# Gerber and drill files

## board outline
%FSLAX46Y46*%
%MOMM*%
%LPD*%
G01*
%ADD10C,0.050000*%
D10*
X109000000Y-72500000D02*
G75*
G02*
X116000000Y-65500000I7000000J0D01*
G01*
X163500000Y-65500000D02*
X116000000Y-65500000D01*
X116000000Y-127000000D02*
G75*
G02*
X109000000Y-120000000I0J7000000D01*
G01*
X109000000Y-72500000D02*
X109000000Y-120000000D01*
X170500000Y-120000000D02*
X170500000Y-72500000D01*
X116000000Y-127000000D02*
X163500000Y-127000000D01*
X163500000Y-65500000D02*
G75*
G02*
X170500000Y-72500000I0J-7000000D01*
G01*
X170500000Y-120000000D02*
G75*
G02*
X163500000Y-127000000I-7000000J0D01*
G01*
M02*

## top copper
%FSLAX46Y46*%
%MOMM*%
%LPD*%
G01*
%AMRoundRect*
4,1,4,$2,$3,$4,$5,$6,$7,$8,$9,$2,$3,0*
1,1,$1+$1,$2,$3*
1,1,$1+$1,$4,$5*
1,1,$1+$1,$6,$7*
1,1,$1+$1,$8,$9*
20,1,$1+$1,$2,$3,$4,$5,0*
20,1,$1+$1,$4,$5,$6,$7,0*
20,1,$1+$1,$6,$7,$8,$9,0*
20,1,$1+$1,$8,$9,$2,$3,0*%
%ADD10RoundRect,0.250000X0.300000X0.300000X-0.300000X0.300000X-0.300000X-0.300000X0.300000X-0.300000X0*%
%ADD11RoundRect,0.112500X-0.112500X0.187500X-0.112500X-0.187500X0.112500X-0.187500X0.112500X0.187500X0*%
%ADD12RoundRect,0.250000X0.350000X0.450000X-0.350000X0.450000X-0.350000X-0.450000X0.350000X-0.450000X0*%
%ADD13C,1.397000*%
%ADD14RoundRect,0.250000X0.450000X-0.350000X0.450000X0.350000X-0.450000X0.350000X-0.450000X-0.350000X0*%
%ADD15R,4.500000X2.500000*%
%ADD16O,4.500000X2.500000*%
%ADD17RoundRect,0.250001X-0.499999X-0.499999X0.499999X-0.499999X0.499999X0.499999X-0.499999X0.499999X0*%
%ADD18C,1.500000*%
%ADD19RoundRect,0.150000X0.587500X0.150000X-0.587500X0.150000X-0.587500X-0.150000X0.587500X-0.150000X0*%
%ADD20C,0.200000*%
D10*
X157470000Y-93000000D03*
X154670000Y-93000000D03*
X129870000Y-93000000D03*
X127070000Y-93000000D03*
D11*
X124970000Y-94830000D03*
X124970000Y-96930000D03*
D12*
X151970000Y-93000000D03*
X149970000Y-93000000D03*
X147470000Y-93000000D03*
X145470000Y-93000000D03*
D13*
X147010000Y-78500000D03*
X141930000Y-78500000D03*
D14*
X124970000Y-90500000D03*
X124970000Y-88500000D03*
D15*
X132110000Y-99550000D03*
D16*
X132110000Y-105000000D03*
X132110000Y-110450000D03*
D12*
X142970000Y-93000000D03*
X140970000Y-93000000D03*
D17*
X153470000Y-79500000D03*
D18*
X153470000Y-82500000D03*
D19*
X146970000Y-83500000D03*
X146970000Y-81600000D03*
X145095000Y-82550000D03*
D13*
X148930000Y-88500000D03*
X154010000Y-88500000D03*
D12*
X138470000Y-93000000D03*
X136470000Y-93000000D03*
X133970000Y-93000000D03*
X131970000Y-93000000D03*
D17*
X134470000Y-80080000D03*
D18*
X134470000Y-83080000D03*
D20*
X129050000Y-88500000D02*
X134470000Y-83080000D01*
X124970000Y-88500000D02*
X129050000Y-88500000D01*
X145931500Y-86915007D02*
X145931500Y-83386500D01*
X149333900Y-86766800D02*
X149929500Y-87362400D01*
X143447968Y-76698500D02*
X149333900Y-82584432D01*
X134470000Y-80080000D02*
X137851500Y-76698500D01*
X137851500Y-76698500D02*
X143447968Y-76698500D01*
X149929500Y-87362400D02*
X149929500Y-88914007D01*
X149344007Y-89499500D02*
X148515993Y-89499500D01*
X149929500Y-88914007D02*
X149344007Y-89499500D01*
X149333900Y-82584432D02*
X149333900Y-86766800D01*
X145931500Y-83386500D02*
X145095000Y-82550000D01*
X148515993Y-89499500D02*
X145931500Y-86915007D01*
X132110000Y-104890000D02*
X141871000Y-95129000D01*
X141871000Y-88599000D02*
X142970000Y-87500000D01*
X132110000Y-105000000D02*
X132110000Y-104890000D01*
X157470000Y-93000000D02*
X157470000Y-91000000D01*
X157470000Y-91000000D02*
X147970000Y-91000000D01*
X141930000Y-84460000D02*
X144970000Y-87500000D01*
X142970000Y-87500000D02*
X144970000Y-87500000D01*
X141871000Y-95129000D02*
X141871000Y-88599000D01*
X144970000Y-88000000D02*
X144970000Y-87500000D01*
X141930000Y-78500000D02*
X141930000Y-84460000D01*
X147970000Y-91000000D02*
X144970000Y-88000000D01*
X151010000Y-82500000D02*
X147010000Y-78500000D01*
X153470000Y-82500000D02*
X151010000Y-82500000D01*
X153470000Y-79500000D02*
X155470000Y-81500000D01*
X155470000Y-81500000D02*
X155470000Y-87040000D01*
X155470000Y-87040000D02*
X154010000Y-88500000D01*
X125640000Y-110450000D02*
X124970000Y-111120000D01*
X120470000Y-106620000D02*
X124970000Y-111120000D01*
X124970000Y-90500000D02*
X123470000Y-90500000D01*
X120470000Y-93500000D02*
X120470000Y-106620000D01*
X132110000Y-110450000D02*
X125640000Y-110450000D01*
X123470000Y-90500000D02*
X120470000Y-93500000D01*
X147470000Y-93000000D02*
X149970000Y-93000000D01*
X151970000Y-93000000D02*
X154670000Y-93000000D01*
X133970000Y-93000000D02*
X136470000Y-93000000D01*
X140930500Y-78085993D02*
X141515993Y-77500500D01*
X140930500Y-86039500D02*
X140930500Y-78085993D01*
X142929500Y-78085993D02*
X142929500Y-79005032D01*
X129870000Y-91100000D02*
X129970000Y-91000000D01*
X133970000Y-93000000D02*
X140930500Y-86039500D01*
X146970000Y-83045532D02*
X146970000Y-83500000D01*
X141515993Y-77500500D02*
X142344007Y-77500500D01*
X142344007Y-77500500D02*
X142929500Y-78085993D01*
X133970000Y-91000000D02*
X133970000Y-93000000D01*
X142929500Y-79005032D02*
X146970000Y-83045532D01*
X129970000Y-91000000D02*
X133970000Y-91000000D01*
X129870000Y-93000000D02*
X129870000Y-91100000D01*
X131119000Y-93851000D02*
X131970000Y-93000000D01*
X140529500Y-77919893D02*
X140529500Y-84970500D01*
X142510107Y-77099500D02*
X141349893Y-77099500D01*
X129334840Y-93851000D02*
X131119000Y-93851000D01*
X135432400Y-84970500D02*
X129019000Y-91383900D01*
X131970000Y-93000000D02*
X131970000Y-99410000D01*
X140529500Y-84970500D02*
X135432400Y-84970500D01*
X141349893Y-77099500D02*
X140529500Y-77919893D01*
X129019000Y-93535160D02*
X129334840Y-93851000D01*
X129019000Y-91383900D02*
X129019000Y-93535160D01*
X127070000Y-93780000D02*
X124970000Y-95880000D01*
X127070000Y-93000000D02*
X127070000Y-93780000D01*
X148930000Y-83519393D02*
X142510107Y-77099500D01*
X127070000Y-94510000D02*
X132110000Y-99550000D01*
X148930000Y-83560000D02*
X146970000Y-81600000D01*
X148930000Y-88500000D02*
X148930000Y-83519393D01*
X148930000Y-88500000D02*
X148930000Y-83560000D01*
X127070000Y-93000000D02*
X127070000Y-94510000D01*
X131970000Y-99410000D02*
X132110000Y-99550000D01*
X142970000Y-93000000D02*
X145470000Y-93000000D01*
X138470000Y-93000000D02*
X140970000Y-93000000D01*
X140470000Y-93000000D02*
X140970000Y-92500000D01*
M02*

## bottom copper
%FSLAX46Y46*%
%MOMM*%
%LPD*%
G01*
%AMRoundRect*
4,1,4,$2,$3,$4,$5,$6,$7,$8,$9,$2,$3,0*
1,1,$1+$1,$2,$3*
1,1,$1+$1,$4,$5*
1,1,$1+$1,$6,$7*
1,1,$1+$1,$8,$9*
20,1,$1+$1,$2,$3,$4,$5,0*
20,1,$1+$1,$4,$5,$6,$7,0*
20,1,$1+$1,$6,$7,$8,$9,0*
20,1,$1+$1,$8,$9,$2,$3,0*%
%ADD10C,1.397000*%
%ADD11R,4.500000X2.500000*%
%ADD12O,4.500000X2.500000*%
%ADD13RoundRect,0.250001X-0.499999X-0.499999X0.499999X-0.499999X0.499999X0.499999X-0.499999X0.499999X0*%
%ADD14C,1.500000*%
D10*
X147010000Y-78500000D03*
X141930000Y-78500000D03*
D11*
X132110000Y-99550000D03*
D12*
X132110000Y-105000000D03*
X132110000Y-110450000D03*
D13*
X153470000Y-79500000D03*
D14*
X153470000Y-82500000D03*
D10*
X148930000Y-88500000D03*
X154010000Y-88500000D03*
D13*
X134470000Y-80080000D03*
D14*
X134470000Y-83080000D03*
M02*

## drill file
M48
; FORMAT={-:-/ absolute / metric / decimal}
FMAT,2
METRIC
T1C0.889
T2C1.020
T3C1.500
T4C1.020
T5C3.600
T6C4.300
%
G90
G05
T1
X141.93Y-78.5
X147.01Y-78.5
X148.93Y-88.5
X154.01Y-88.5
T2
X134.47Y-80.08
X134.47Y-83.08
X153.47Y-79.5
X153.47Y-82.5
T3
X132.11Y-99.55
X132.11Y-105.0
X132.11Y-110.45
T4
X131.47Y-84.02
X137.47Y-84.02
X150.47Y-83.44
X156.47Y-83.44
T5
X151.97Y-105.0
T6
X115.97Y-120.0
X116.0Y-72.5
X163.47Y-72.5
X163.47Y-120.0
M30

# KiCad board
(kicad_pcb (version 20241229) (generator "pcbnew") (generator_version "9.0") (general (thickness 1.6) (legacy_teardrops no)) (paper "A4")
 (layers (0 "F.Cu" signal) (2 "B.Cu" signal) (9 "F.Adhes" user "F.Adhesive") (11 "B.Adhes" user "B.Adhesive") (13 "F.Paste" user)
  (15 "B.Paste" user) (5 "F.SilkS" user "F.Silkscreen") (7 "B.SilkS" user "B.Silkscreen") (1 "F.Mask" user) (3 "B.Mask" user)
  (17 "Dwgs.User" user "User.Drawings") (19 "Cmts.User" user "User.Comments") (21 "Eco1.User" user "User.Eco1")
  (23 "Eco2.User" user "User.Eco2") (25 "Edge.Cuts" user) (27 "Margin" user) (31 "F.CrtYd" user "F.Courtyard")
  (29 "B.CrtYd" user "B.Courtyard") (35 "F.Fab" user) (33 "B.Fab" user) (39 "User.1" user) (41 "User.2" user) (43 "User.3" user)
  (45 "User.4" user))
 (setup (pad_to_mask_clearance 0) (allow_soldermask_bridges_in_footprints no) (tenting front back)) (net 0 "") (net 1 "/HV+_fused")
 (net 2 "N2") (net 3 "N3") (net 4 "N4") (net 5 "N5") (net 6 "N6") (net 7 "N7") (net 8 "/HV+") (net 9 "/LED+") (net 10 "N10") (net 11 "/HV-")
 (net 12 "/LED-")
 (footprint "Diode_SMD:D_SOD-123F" (layer "F.Cu") (at 156.07 93 180)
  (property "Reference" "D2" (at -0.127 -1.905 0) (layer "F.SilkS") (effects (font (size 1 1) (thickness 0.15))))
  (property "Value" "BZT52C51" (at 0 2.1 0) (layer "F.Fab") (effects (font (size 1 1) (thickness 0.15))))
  (pad "1" smd roundrect (at -1.4 0 180) (size 1.1 1.1) (layers "F.Cu" "F.Mask" "F.Paste") (roundrect_rratio 0.2272727273)
   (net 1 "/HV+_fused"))
  (pad "2" smd roundrect (at 1.4 0 180) (size 1.1 1.1) (layers "F.Cu" "F.Mask" "F.Paste") (roundrect_rratio 0.2272727273) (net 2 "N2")))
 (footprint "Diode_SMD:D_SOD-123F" (layer "F.Cu") (at 128.47 93 180)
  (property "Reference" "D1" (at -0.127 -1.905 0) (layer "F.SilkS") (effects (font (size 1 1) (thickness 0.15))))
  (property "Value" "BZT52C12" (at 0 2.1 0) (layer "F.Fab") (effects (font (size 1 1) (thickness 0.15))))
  (pad "1" smd roundrect (at -1.4 0 180) (size 1.1 1.1) (layers "F.Cu" "F.Mask" "F.Paste") (roundrect_rratio 0.2272727273) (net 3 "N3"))
  (pad "2" smd roundrect (at 1.4 0 180) (size 1.1 1.1) (layers "F.Cu" "F.Mask" "F.Paste") (roundrect_rratio 0.2272727273) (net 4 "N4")))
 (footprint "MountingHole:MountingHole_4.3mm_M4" (layer "F.Cu") (at 116 72.5)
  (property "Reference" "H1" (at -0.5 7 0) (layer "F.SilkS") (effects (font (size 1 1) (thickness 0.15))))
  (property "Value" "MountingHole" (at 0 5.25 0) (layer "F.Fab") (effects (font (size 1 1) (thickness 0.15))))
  (pad "" np_thru_hole circle (at 0 0) (size 4.3 4.3) (drill 4.3) (layers "*.Cu" "*.Mask")))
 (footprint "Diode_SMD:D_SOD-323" (layer "F.Cu") (at 124.97 95.88 -90)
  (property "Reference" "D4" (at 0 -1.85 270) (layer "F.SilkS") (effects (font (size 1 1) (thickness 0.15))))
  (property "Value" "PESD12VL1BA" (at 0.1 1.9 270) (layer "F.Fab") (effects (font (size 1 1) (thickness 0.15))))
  (pad "1" smd roundrect (at -1.05 0 270) (size 0.6 0.45) (layers "F.Cu" "F.Mask" "F.Paste") (roundrect_rratio 0.25) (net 4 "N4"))
  (pad "2" smd roundrect (at 1.05 0 270) (size 0.6 0.45) (layers "F.Cu" "F.Mask" "F.Paste") (roundrect_rratio 0.25) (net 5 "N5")))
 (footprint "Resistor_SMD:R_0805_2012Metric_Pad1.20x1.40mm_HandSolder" (layer "F.Cu") (at 150.97 93 180)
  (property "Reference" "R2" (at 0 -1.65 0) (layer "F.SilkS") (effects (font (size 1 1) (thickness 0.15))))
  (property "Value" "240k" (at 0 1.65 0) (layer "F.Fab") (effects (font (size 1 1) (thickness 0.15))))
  (pad "1" smd roundrect (at -1 0 180) (size 1.2 1.4) (layers "F.Cu" "F.Mask" "F.Paste") (roundrect_rratio 0.208333) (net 2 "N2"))
  (pad "2" smd roundrect (at 1 0 180) (size 1.2 1.4) (layers "F.Cu" "F.Mask" "F.Paste") (roundrect_rratio 0.208333) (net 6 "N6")))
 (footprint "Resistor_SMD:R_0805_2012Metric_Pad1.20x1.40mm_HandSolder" (layer "F.Cu") (at 146.47 93 180)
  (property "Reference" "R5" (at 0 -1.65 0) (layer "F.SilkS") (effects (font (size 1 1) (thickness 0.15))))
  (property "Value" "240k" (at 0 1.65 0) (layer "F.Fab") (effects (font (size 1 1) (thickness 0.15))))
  (pad "1" smd roundrect (at -1 0 180) (size 1.2 1.4) (layers "F.Cu" "F.Mask" "F.Paste") (roundrect_rratio 0.208333) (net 6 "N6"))
  (pad "2" smd roundrect (at 1 0 180) (size 1.2 1.4) (layers "F.Cu" "F.Mask" "F.Paste") (roundrect_rratio 0.208333) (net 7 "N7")))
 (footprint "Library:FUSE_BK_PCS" (layer "F.Cu") (at 144.47 78.5 180)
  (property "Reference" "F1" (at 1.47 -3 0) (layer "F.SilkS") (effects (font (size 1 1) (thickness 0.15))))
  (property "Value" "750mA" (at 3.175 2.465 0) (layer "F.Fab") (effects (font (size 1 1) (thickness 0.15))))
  (pad "1" thru_hole circle (at -2.54 0 180) (size 1.397 1.397) (drill 0.889) (layers "*.Cu" "*.Mask") (remove_unused_layers no)
   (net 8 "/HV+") (solder_mask_margin 0.102))
  (pad "2" thru_hole circle (at 2.54 0 180) (size 1.397 1.397) (drill 0.889) (layers "*.Cu" "*.Mask") (remove_unused_layers no)
   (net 1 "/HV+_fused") (solder_mask_margin 0.102)))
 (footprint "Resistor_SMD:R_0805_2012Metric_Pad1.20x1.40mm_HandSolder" (layer "F.Cu") (at 124.97 89.5 90)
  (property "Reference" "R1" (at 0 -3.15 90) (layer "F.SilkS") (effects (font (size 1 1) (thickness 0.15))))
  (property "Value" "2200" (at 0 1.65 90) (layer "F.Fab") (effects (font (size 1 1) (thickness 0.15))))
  (pad "1" smd roundrect (at -1 0 90) (size 1.2 1.4) (layers "F.Cu" "F.Mask" "F.Paste") (roundrect_rratio 0.208333) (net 5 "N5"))
  (pad "2" smd roundrect (at 1 0 90) (size 1.2 1.4) (layers "F.Cu" "F.Mask" "F.Paste") (roundrect_rratio 0.208333) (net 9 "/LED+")))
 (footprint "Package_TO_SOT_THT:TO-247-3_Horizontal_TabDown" (layer "F.Cu") (at 132.11 99.55 -90)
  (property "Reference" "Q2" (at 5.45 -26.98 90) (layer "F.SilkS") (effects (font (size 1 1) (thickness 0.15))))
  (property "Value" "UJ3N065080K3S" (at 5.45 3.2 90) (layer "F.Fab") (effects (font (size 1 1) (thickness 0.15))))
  (pad "" np_thru_hole circle (at 5.45 -19.86 270) (size 3.6 3.6) (drill 3.6) (layers "*.Cu" "*.Mask"))
  (pad "1" thru_hole rect (at 0 0 270) (size 2.5 4.5) (drill 1.5) (layers "*.Cu" "*.Mask") (remove_unused_layers no) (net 4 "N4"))
  (pad "2" thru_hole oval (at 5.45 0 270) (size 2.5 4.5) (drill 1.5) (layers "*.Cu" "*.Mask") (remove_unused_layers no) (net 1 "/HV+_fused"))
  (pad "3" thru_hole oval (at 10.9 0 270) (size 2.5 4.5) (drill 1.5) (layers "*.Cu" "*.Mask") (remove_unused_layers no) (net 5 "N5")))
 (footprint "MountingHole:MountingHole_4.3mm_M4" (layer "F.Cu") (at 115.97 120)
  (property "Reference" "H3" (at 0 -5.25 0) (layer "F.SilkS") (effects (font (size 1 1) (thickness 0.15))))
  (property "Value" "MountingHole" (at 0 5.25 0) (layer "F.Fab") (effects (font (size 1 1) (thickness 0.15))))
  (pad "" np_thru_hole circle (at 0 0) (size 4.3 4.3) (drill 4.3) (layers "*.Cu" "*.Mask")))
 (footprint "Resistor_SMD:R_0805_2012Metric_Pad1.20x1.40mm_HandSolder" (layer "F.Cu") (at 141.97 93 180)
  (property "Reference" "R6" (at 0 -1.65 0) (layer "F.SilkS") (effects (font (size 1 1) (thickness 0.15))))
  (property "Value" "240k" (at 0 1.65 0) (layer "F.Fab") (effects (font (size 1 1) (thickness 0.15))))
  (pad "1" smd roundrect (at -1 0 180) (size 1.2 1.4) (layers "F.Cu" "F.Mask" "F.Paste") (roundrect_rratio 0.208333) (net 7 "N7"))
  (pad "2" smd roundrect (at 1 0 180) (size 1.2 1.4) (layers "F.Cu" "F.Mask" "F.Paste") (roundrect_rratio 0.208333) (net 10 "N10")))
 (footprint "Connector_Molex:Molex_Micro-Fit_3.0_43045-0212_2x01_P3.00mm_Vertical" (layer "F.Cu") (at 153.47 79.5)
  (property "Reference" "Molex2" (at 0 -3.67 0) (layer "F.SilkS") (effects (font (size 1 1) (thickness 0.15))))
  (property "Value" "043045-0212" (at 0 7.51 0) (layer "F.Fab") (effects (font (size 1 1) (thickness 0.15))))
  (pad "" np_thru_hole circle (at -3 3.94) (size 1.02 1.02) (drill 1.02) (layers "*.Cu" "*.Mask"))
  (pad "" np_thru_hole circle (at 3 3.94) (size 1.02 1.02) (drill 1.02) (layers "*.Cu" "*.Mask"))
  (pad "1" thru_hole roundrect (at 0 0) (size 1.5 1.5) (drill 1.02) (layers "*.Cu" "*.Mask") (remove_unused_layers no)
   (roundrect_rratio 0.166667) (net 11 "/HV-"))
  (pad "2" thru_hole circle (at 0 3) (size 1.5 1.5) (drill 1.02) (layers "*.Cu" "*.Mask") (remove_unused_layers no) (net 8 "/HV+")))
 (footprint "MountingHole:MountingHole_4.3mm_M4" (layer "F.Cu") (at 163.47 72.5)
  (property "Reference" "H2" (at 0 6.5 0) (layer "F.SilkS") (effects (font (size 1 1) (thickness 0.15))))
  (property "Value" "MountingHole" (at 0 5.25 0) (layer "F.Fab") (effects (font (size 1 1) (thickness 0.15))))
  (pad "" np_thru_hole circle (at 0 0) (size 4.3 4.3) (drill 4.3) (layers "*.Cu" "*.Mask")))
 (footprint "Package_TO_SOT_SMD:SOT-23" (layer "F.Cu") (at 146.0325 82.55 180)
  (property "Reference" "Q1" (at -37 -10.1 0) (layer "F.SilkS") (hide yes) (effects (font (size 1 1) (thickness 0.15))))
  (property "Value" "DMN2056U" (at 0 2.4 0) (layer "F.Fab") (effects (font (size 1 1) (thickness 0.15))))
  (pad "1" smd roundrect (at -0.9375 -0.95 180) (size 1.475 0.6) (layers "F.Cu" "F.Mask" "F.Paste") (roundrect_rratio 0.25) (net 3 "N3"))
  (pad "2" smd roundrect (at -0.9375 0.95 180) (size 1.475 0.6) (layers "F.Cu" "F.Mask" "F.Paste") (roundrect_rratio 0.25) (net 4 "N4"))
  (pad "3" smd roundrect (at 0.9375 0 180) (size 1.475 0.6) (layers "F.Cu" "F.Mask" "F.Paste") (roundrect_rratio 0.25) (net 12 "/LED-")))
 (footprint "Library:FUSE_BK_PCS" (layer "F.Cu") (at 151.47 88.5)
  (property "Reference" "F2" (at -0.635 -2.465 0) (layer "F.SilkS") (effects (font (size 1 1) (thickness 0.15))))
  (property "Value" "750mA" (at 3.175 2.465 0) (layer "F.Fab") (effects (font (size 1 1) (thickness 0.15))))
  (pad "1" thru_hole circle (at -2.54 0) (size 1.397 1.397) (drill 0.889) (layers "*.Cu" "*.Mask") (remove_unused_layers no) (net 4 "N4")
   (solder_mask_margin 0.102))
  (pad "2" thru_hole circle (at 2.54 0) (size 1.397 1.397) (drill 0.889) (layers "*.Cu" "*.Mask") (remove_unused_layers no) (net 11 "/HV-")
   (solder_mask_margin 0.102)))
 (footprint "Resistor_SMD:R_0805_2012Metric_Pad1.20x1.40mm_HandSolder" (layer "F.Cu") (at 137.47 93 180)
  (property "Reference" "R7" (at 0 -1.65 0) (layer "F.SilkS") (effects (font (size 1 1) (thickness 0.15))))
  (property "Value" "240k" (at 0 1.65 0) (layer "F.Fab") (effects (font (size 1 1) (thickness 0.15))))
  (pad "1" smd roundrect (at -1 0 180) (size 1.2 1.4) (layers "F.Cu" "F.Mask" "F.Paste") (roundrect_rratio 0.208333) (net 10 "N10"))
  (pad "2" smd roundrect (at 1 0 180) (size 1.2 1.4) (layers "F.Cu" "F.Mask" "F.Paste") (roundrect_rratio 0.208333) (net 3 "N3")))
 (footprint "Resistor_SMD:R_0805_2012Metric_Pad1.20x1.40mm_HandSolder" (layer "F.Cu") (at 132.97 93 180)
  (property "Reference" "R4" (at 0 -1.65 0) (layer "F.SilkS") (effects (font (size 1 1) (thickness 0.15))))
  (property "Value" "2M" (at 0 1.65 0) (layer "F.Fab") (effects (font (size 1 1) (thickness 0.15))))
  (pad "1" smd roundrect (at -1 0 180) (size 1.2 1.4) (layers "F.Cu" "F.Mask" "F.Paste") (roundrect_rratio 0.208333) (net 3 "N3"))
  (pad "2" smd roundrect (at 1 0 180) (size 1.2 1.4) (layers "F.Cu" "F.Mask" "F.Paste") (roundrect_rratio 0.208333) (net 4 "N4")))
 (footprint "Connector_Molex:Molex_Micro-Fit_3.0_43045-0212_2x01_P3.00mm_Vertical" (layer "F.Cu") (at 134.47 80.08)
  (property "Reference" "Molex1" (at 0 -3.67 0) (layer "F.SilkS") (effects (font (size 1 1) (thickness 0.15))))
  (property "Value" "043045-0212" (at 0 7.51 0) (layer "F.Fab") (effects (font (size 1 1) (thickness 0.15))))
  (pad "" np_thru_hole circle (at -3 3.94) (size 1.02 1.02) (drill 1.02) (layers "*.Cu" "*.Mask"))
  (pad "" np_thru_hole circle (at 3 3.94) (size 1.02 1.02) (drill 1.02) (layers "*.Cu" "*.Mask"))
  (pad "1" thru_hole roundrect (at 0 0) (size 1.5 1.5) (drill 1.02) (layers "*.Cu" "*.Mask") (remove_unused_layers no)
   (roundrect_rratio 0.166667) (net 12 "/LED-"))
  (pad "2" thru_hole circle (at 0 3) (size 1.5 1.5) (drill 1.02) (layers "*.Cu" "*.Mask") (remove_unused_layers no) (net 9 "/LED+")))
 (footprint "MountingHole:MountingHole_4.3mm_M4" (layer "F.Cu") (at 163.47 120)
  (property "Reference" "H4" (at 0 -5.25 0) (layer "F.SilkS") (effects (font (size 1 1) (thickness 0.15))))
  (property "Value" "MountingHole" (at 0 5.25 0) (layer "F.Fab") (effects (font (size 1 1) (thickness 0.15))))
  (pad "" np_thru_hole circle (at 0 0) (size 4.3 4.3) (drill 4.3) (layers "*.Cu" "*.Mask")))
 (gr_arc (start 109 72.5) (mid 111.050253 67.550253) (end 116 65.5) (stroke (width 0.05) (type default)) (layer "Edge.Cuts"))
 (gr_line (start 163.5 65.5) (end 116 65.5) (stroke (width 0.05) (type default)) (layer "Edge.Cuts"))
 (gr_arc (start 116 127) (mid 111.050253 124.949747) (end 109 120) (stroke (width 0.05) (type default)) (layer "Edge.Cuts"))
 (gr_line (start 109 72.5) (end 109 120) (stroke (width 0.05) (type default)) (layer "Edge.Cuts"))
 (gr_line (start 170.5 120) (end 170.5 72.5) (stroke (width 0.05) (type default)) (layer "Edge.Cuts"))
 (gr_line (start 116 127) (end 163.5 127) (stroke (width 0.05) (type default)) (layer "Edge.Cuts"))
 (gr_arc (start 163.5 65.5) (mid 168.449747 67.550253) (end 170.5 72.5) (stroke (width 0.05) (type default)) (layer "Edge.Cuts"))
 (gr_arc (start 170.5 120) (mid 168.449747 124.949747) (end 163.5 127) (stroke (width 0.05) (type default)) (layer "Edge.Cuts"))
 (segment (start 129.05 88.5) (end 134.47 83.08) (width 0.2) (layer "F.Cu") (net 9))
 (segment (start 124.97 88.5) (end 129.05 88.5) (width 0.2) (layer "F.Cu") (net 9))
 (segment (start 145.9315 86.915007) (end 145.9315 83.3865) (width 0.2) (layer "F.Cu") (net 12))
 (segment (start 149.3339 86.7668) (end 149.9295 87.3624) (width 0.2) (layer "F.Cu") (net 12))
 (segment (start 143.447968 76.6985) (end 149.3339 82.584432) (width 0.2) (layer "F.Cu") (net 12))
 (segment (start 134.47 80.08) (end 137.8515 76.6985) (width 0.2) (layer "F.Cu") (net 12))
 (segment (start 137.8515 76.6985) (end 143.447968 76.6985) (width 0.2) (layer "F.Cu") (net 12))
 (segment (start 149.9295 87.3624) (end 149.9295 88.914007) (width 0.2) (layer "F.Cu") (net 12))
 (segment (start 149.344007 89.4995) (end 148.515993 89.4995) (width 0.2) (layer "F.Cu") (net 12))
 (segment (start 149.9295 88.914007) (end 149.344007 89.4995) (width 0.2) (layer "F.Cu") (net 12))
 (segment (start 149.3339 82.584432) (end 149.3339 86.7668) (width 0.2) (layer "F.Cu") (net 12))
 (segment (start 145.9315 83.3865) (end 145.095 82.55) (width 0.2) (layer "F.Cu") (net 12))
 (segment (start 148.515993 89.4995) (end 145.9315 86.915007) (width 0.2) (layer "F.Cu") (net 12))
 (segment (start 132.11 104.89) (end 141.871 95.129) (width 0.2) (layer "F.Cu") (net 1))
 (segment (start 141.871 88.599) (end 142.97 87.5) (width 0.2) (layer "F.Cu") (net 1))
 (segment (start 132.11 105) (end 132.11 104.89) (width 0.2) (layer "F.Cu") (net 1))
 (segment (start 157.47 93) (end 157.47 91) (width 0.2) (layer "F.Cu") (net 1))
 (segment (start 157.47 91) (end 147.97 91) (width 0.2) (layer "F.Cu") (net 1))
 (segment (start 141.93 84.46) (end 144.97 87.5) (width 0.2) (layer "F.Cu") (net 1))
 (segment (start 142.97 87.5) (end 144.97 87.5) (width 0.2) (layer "F.Cu") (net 1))
 (segment (start 141.871 95.129) (end 141.871 88.599) (width 0.2) (layer "F.Cu") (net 1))
 (segment (start 144.97 88) (end 144.97 87.5) (width 0.2) (layer "F.Cu") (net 1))
 (segment (start 141.93 78.5) (end 141.93 84.46) (width 0.2) (layer "F.Cu") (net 1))
 (segment (start 147.97 91) (end 144.97 88) (width 0.2) (layer "F.Cu") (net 1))
 (segment (start 151.01 82.5) (end 147.01 78.5) (width 0.2) (layer "F.Cu") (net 8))
 (segment (start 153.47 82.5) (end 151.01 82.5) (width 0.2) (layer "F.Cu") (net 8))
 (segment (start 153.47 79.5) (end 155.47 81.5) (width 0.2) (layer "F.Cu") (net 11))
 (segment (start 155.47 81.5) (end 155.47 87.04) (width 0.2) (layer "F.Cu") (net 11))
 (segment (start 155.47 87.04) (end 154.01 88.5) (width 0.2) (layer "F.Cu") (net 11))
 (segment (start 125.64 110.45) (end 124.97 111.12) (width 0.2) (layer "F.Cu") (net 5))
 (segment (start 120.47 106.62) (end 124.97 111.12) (width 0.2) (layer "F.Cu") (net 5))
 (segment (start 124.97 90.5) (end 123.47 90.5) (width 0.2) (layer "F.Cu") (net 5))
 (segment (start 120.47 93.5) (end 120.47 106.62) (width 0.2) (layer "F.Cu") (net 5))
 (segment (start 132.11 110.45) (end 125.64 110.45) (width 0.2) (layer "F.Cu") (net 5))
 (segment (start 123.47 90.5) (end 120.47 93.5) (width 0.2) (layer "F.Cu") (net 5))
 (segment (start 147.47 93) (end 149.97 93) (width 0.2) (layer "F.Cu") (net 6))
 (segment (start 151.97 93) (end 154.67 93) (width 0.2) (layer "F.Cu") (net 2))
 (segment (start 133.97 93) (end 136.47 93) (width 0.2) (layer "F.Cu") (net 3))
 (segment (start 140.9305 78.085993) (end 141.515993 77.5005) (width 0.2) (layer "F.Cu") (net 3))
 (segment (start 140.9305 86.0395) (end 140.9305 78.085993) (width 0.2) (layer "F.Cu") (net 3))
 (segment (start 142.9295 78.085993) (end 142.9295 79.005032) (width 0.2) (layer "F.Cu") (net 3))
 (segment (start 129.87 91.1) (end 129.97 91) (width 0.2) (layer "F.Cu") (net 3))
 (segment (start 133.97 93) (end 140.9305 86.0395) (width 0.2) (layer "F.Cu") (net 3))
 (segment (start 146.97 83.045532) (end 146.97 83.5) (width 0.2) (layer "F.Cu") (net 3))
 (segment (start 141.515993 77.5005) (end 142.344007 77.5005) (width 0.2) (layer "F.Cu") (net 3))
 (segment (start 142.344007 77.5005) (end 142.9295 78.085993) (width 0.2) (layer "F.Cu") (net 3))
 (segment (start 133.97 91) (end 133.97 93) (width 0.2) (layer "F.Cu") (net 3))
 (segment (start 142.9295 79.005032) (end 146.97 83.045532) (width 0.2) (layer "F.Cu") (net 3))
 (segment (start 129.97 91) (end 133.97 91) (width 0.2) (layer "F.Cu") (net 3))
 (segment (start 129.87 93) (end 129.87 91.1) (width 0.2) (layer "F.Cu") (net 3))
 (segment (start 131.119 93.851) (end 131.97 93) (width 0.2) (layer "F.Cu") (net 4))
 (segment (start 140.5295 77.919893) (end 140.5295 84.9705) (width 0.2) (layer "F.Cu") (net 4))
 (segment (start 142.510107 77.0995) (end 141.349893 77.0995) (width 0.2) (layer "F.Cu") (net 4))
 (segment (start 129.33484 93.851) (end 131.119 93.851) (width 0.2) (layer "F.Cu") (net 4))
 (segment (start 135.4324 84.9705) (end 129.019 91.3839) (width 0.2) (layer "F.Cu") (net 4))
 (segment (start 131.97 93) (end 131.97 99.41) (width 0.2) (layer "F.Cu") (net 4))
 (segment (start 140.5295 84.9705) (end 135.4324 84.9705) (width 0.2) (layer "F.Cu") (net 4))
 (segment (start 141.349893 77.0995) (end 140.5295 77.919893) (width 0.2) (layer "F.Cu") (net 4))
 (segment (start 129.019 93.53516) (end 129.33484 93.851) (width 0.2) (layer "F.Cu") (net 4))
 (segment (start 129.019 91.3839) (end 129.019 93.53516) (width 0.2) (layer "F.Cu") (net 4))
 (segment (start 127.07 93.78) (end 124.97 95.88) (width 0.2) (layer "F.Cu") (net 4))
 (segment (start 127.07 93) (end 127.07 93.78) (width 0.2) (layer "F.Cu") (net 4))
 (segment (start 148.93 83.519393) (end 142.510107 77.0995) (width 0.2) (layer "F.Cu") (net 4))
 (segment (start 127.07 94.51) (end 132.11 99.55) (width 0.2) (layer "F.Cu") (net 4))
 (segment (start 148.93 83.56) (end 146.97 81.6) (width 0.2) (layer "F.Cu") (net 4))
 (segment (start 148.93 88.5) (end 148.93 83.519393) (width 0.2) (layer "F.Cu") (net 4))
 (segment (start 148.93 88.5) (end 148.93 83.56) (width 0.2) (layer "F.Cu") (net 4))
 (segment (start 127.07 93) (end 127.07 94.51) (width 0.2) (layer "F.Cu") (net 4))
 (segment (start 131.97 99.41) (end 132.11 99.55) (width 0.2) (layer "F.Cu") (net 4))
 (segment (start 142.97 93) (end 145.47 93) (width 0.2) (layer "F.Cu") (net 7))
 (segment (start 138.47 93) (end 140.97 93) (width 0.2) (layer "F.Cu") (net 10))
 (segment (start 140.47 93) (end 140.97 92.5) (width 0.2) (layer "F.Cu") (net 10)))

